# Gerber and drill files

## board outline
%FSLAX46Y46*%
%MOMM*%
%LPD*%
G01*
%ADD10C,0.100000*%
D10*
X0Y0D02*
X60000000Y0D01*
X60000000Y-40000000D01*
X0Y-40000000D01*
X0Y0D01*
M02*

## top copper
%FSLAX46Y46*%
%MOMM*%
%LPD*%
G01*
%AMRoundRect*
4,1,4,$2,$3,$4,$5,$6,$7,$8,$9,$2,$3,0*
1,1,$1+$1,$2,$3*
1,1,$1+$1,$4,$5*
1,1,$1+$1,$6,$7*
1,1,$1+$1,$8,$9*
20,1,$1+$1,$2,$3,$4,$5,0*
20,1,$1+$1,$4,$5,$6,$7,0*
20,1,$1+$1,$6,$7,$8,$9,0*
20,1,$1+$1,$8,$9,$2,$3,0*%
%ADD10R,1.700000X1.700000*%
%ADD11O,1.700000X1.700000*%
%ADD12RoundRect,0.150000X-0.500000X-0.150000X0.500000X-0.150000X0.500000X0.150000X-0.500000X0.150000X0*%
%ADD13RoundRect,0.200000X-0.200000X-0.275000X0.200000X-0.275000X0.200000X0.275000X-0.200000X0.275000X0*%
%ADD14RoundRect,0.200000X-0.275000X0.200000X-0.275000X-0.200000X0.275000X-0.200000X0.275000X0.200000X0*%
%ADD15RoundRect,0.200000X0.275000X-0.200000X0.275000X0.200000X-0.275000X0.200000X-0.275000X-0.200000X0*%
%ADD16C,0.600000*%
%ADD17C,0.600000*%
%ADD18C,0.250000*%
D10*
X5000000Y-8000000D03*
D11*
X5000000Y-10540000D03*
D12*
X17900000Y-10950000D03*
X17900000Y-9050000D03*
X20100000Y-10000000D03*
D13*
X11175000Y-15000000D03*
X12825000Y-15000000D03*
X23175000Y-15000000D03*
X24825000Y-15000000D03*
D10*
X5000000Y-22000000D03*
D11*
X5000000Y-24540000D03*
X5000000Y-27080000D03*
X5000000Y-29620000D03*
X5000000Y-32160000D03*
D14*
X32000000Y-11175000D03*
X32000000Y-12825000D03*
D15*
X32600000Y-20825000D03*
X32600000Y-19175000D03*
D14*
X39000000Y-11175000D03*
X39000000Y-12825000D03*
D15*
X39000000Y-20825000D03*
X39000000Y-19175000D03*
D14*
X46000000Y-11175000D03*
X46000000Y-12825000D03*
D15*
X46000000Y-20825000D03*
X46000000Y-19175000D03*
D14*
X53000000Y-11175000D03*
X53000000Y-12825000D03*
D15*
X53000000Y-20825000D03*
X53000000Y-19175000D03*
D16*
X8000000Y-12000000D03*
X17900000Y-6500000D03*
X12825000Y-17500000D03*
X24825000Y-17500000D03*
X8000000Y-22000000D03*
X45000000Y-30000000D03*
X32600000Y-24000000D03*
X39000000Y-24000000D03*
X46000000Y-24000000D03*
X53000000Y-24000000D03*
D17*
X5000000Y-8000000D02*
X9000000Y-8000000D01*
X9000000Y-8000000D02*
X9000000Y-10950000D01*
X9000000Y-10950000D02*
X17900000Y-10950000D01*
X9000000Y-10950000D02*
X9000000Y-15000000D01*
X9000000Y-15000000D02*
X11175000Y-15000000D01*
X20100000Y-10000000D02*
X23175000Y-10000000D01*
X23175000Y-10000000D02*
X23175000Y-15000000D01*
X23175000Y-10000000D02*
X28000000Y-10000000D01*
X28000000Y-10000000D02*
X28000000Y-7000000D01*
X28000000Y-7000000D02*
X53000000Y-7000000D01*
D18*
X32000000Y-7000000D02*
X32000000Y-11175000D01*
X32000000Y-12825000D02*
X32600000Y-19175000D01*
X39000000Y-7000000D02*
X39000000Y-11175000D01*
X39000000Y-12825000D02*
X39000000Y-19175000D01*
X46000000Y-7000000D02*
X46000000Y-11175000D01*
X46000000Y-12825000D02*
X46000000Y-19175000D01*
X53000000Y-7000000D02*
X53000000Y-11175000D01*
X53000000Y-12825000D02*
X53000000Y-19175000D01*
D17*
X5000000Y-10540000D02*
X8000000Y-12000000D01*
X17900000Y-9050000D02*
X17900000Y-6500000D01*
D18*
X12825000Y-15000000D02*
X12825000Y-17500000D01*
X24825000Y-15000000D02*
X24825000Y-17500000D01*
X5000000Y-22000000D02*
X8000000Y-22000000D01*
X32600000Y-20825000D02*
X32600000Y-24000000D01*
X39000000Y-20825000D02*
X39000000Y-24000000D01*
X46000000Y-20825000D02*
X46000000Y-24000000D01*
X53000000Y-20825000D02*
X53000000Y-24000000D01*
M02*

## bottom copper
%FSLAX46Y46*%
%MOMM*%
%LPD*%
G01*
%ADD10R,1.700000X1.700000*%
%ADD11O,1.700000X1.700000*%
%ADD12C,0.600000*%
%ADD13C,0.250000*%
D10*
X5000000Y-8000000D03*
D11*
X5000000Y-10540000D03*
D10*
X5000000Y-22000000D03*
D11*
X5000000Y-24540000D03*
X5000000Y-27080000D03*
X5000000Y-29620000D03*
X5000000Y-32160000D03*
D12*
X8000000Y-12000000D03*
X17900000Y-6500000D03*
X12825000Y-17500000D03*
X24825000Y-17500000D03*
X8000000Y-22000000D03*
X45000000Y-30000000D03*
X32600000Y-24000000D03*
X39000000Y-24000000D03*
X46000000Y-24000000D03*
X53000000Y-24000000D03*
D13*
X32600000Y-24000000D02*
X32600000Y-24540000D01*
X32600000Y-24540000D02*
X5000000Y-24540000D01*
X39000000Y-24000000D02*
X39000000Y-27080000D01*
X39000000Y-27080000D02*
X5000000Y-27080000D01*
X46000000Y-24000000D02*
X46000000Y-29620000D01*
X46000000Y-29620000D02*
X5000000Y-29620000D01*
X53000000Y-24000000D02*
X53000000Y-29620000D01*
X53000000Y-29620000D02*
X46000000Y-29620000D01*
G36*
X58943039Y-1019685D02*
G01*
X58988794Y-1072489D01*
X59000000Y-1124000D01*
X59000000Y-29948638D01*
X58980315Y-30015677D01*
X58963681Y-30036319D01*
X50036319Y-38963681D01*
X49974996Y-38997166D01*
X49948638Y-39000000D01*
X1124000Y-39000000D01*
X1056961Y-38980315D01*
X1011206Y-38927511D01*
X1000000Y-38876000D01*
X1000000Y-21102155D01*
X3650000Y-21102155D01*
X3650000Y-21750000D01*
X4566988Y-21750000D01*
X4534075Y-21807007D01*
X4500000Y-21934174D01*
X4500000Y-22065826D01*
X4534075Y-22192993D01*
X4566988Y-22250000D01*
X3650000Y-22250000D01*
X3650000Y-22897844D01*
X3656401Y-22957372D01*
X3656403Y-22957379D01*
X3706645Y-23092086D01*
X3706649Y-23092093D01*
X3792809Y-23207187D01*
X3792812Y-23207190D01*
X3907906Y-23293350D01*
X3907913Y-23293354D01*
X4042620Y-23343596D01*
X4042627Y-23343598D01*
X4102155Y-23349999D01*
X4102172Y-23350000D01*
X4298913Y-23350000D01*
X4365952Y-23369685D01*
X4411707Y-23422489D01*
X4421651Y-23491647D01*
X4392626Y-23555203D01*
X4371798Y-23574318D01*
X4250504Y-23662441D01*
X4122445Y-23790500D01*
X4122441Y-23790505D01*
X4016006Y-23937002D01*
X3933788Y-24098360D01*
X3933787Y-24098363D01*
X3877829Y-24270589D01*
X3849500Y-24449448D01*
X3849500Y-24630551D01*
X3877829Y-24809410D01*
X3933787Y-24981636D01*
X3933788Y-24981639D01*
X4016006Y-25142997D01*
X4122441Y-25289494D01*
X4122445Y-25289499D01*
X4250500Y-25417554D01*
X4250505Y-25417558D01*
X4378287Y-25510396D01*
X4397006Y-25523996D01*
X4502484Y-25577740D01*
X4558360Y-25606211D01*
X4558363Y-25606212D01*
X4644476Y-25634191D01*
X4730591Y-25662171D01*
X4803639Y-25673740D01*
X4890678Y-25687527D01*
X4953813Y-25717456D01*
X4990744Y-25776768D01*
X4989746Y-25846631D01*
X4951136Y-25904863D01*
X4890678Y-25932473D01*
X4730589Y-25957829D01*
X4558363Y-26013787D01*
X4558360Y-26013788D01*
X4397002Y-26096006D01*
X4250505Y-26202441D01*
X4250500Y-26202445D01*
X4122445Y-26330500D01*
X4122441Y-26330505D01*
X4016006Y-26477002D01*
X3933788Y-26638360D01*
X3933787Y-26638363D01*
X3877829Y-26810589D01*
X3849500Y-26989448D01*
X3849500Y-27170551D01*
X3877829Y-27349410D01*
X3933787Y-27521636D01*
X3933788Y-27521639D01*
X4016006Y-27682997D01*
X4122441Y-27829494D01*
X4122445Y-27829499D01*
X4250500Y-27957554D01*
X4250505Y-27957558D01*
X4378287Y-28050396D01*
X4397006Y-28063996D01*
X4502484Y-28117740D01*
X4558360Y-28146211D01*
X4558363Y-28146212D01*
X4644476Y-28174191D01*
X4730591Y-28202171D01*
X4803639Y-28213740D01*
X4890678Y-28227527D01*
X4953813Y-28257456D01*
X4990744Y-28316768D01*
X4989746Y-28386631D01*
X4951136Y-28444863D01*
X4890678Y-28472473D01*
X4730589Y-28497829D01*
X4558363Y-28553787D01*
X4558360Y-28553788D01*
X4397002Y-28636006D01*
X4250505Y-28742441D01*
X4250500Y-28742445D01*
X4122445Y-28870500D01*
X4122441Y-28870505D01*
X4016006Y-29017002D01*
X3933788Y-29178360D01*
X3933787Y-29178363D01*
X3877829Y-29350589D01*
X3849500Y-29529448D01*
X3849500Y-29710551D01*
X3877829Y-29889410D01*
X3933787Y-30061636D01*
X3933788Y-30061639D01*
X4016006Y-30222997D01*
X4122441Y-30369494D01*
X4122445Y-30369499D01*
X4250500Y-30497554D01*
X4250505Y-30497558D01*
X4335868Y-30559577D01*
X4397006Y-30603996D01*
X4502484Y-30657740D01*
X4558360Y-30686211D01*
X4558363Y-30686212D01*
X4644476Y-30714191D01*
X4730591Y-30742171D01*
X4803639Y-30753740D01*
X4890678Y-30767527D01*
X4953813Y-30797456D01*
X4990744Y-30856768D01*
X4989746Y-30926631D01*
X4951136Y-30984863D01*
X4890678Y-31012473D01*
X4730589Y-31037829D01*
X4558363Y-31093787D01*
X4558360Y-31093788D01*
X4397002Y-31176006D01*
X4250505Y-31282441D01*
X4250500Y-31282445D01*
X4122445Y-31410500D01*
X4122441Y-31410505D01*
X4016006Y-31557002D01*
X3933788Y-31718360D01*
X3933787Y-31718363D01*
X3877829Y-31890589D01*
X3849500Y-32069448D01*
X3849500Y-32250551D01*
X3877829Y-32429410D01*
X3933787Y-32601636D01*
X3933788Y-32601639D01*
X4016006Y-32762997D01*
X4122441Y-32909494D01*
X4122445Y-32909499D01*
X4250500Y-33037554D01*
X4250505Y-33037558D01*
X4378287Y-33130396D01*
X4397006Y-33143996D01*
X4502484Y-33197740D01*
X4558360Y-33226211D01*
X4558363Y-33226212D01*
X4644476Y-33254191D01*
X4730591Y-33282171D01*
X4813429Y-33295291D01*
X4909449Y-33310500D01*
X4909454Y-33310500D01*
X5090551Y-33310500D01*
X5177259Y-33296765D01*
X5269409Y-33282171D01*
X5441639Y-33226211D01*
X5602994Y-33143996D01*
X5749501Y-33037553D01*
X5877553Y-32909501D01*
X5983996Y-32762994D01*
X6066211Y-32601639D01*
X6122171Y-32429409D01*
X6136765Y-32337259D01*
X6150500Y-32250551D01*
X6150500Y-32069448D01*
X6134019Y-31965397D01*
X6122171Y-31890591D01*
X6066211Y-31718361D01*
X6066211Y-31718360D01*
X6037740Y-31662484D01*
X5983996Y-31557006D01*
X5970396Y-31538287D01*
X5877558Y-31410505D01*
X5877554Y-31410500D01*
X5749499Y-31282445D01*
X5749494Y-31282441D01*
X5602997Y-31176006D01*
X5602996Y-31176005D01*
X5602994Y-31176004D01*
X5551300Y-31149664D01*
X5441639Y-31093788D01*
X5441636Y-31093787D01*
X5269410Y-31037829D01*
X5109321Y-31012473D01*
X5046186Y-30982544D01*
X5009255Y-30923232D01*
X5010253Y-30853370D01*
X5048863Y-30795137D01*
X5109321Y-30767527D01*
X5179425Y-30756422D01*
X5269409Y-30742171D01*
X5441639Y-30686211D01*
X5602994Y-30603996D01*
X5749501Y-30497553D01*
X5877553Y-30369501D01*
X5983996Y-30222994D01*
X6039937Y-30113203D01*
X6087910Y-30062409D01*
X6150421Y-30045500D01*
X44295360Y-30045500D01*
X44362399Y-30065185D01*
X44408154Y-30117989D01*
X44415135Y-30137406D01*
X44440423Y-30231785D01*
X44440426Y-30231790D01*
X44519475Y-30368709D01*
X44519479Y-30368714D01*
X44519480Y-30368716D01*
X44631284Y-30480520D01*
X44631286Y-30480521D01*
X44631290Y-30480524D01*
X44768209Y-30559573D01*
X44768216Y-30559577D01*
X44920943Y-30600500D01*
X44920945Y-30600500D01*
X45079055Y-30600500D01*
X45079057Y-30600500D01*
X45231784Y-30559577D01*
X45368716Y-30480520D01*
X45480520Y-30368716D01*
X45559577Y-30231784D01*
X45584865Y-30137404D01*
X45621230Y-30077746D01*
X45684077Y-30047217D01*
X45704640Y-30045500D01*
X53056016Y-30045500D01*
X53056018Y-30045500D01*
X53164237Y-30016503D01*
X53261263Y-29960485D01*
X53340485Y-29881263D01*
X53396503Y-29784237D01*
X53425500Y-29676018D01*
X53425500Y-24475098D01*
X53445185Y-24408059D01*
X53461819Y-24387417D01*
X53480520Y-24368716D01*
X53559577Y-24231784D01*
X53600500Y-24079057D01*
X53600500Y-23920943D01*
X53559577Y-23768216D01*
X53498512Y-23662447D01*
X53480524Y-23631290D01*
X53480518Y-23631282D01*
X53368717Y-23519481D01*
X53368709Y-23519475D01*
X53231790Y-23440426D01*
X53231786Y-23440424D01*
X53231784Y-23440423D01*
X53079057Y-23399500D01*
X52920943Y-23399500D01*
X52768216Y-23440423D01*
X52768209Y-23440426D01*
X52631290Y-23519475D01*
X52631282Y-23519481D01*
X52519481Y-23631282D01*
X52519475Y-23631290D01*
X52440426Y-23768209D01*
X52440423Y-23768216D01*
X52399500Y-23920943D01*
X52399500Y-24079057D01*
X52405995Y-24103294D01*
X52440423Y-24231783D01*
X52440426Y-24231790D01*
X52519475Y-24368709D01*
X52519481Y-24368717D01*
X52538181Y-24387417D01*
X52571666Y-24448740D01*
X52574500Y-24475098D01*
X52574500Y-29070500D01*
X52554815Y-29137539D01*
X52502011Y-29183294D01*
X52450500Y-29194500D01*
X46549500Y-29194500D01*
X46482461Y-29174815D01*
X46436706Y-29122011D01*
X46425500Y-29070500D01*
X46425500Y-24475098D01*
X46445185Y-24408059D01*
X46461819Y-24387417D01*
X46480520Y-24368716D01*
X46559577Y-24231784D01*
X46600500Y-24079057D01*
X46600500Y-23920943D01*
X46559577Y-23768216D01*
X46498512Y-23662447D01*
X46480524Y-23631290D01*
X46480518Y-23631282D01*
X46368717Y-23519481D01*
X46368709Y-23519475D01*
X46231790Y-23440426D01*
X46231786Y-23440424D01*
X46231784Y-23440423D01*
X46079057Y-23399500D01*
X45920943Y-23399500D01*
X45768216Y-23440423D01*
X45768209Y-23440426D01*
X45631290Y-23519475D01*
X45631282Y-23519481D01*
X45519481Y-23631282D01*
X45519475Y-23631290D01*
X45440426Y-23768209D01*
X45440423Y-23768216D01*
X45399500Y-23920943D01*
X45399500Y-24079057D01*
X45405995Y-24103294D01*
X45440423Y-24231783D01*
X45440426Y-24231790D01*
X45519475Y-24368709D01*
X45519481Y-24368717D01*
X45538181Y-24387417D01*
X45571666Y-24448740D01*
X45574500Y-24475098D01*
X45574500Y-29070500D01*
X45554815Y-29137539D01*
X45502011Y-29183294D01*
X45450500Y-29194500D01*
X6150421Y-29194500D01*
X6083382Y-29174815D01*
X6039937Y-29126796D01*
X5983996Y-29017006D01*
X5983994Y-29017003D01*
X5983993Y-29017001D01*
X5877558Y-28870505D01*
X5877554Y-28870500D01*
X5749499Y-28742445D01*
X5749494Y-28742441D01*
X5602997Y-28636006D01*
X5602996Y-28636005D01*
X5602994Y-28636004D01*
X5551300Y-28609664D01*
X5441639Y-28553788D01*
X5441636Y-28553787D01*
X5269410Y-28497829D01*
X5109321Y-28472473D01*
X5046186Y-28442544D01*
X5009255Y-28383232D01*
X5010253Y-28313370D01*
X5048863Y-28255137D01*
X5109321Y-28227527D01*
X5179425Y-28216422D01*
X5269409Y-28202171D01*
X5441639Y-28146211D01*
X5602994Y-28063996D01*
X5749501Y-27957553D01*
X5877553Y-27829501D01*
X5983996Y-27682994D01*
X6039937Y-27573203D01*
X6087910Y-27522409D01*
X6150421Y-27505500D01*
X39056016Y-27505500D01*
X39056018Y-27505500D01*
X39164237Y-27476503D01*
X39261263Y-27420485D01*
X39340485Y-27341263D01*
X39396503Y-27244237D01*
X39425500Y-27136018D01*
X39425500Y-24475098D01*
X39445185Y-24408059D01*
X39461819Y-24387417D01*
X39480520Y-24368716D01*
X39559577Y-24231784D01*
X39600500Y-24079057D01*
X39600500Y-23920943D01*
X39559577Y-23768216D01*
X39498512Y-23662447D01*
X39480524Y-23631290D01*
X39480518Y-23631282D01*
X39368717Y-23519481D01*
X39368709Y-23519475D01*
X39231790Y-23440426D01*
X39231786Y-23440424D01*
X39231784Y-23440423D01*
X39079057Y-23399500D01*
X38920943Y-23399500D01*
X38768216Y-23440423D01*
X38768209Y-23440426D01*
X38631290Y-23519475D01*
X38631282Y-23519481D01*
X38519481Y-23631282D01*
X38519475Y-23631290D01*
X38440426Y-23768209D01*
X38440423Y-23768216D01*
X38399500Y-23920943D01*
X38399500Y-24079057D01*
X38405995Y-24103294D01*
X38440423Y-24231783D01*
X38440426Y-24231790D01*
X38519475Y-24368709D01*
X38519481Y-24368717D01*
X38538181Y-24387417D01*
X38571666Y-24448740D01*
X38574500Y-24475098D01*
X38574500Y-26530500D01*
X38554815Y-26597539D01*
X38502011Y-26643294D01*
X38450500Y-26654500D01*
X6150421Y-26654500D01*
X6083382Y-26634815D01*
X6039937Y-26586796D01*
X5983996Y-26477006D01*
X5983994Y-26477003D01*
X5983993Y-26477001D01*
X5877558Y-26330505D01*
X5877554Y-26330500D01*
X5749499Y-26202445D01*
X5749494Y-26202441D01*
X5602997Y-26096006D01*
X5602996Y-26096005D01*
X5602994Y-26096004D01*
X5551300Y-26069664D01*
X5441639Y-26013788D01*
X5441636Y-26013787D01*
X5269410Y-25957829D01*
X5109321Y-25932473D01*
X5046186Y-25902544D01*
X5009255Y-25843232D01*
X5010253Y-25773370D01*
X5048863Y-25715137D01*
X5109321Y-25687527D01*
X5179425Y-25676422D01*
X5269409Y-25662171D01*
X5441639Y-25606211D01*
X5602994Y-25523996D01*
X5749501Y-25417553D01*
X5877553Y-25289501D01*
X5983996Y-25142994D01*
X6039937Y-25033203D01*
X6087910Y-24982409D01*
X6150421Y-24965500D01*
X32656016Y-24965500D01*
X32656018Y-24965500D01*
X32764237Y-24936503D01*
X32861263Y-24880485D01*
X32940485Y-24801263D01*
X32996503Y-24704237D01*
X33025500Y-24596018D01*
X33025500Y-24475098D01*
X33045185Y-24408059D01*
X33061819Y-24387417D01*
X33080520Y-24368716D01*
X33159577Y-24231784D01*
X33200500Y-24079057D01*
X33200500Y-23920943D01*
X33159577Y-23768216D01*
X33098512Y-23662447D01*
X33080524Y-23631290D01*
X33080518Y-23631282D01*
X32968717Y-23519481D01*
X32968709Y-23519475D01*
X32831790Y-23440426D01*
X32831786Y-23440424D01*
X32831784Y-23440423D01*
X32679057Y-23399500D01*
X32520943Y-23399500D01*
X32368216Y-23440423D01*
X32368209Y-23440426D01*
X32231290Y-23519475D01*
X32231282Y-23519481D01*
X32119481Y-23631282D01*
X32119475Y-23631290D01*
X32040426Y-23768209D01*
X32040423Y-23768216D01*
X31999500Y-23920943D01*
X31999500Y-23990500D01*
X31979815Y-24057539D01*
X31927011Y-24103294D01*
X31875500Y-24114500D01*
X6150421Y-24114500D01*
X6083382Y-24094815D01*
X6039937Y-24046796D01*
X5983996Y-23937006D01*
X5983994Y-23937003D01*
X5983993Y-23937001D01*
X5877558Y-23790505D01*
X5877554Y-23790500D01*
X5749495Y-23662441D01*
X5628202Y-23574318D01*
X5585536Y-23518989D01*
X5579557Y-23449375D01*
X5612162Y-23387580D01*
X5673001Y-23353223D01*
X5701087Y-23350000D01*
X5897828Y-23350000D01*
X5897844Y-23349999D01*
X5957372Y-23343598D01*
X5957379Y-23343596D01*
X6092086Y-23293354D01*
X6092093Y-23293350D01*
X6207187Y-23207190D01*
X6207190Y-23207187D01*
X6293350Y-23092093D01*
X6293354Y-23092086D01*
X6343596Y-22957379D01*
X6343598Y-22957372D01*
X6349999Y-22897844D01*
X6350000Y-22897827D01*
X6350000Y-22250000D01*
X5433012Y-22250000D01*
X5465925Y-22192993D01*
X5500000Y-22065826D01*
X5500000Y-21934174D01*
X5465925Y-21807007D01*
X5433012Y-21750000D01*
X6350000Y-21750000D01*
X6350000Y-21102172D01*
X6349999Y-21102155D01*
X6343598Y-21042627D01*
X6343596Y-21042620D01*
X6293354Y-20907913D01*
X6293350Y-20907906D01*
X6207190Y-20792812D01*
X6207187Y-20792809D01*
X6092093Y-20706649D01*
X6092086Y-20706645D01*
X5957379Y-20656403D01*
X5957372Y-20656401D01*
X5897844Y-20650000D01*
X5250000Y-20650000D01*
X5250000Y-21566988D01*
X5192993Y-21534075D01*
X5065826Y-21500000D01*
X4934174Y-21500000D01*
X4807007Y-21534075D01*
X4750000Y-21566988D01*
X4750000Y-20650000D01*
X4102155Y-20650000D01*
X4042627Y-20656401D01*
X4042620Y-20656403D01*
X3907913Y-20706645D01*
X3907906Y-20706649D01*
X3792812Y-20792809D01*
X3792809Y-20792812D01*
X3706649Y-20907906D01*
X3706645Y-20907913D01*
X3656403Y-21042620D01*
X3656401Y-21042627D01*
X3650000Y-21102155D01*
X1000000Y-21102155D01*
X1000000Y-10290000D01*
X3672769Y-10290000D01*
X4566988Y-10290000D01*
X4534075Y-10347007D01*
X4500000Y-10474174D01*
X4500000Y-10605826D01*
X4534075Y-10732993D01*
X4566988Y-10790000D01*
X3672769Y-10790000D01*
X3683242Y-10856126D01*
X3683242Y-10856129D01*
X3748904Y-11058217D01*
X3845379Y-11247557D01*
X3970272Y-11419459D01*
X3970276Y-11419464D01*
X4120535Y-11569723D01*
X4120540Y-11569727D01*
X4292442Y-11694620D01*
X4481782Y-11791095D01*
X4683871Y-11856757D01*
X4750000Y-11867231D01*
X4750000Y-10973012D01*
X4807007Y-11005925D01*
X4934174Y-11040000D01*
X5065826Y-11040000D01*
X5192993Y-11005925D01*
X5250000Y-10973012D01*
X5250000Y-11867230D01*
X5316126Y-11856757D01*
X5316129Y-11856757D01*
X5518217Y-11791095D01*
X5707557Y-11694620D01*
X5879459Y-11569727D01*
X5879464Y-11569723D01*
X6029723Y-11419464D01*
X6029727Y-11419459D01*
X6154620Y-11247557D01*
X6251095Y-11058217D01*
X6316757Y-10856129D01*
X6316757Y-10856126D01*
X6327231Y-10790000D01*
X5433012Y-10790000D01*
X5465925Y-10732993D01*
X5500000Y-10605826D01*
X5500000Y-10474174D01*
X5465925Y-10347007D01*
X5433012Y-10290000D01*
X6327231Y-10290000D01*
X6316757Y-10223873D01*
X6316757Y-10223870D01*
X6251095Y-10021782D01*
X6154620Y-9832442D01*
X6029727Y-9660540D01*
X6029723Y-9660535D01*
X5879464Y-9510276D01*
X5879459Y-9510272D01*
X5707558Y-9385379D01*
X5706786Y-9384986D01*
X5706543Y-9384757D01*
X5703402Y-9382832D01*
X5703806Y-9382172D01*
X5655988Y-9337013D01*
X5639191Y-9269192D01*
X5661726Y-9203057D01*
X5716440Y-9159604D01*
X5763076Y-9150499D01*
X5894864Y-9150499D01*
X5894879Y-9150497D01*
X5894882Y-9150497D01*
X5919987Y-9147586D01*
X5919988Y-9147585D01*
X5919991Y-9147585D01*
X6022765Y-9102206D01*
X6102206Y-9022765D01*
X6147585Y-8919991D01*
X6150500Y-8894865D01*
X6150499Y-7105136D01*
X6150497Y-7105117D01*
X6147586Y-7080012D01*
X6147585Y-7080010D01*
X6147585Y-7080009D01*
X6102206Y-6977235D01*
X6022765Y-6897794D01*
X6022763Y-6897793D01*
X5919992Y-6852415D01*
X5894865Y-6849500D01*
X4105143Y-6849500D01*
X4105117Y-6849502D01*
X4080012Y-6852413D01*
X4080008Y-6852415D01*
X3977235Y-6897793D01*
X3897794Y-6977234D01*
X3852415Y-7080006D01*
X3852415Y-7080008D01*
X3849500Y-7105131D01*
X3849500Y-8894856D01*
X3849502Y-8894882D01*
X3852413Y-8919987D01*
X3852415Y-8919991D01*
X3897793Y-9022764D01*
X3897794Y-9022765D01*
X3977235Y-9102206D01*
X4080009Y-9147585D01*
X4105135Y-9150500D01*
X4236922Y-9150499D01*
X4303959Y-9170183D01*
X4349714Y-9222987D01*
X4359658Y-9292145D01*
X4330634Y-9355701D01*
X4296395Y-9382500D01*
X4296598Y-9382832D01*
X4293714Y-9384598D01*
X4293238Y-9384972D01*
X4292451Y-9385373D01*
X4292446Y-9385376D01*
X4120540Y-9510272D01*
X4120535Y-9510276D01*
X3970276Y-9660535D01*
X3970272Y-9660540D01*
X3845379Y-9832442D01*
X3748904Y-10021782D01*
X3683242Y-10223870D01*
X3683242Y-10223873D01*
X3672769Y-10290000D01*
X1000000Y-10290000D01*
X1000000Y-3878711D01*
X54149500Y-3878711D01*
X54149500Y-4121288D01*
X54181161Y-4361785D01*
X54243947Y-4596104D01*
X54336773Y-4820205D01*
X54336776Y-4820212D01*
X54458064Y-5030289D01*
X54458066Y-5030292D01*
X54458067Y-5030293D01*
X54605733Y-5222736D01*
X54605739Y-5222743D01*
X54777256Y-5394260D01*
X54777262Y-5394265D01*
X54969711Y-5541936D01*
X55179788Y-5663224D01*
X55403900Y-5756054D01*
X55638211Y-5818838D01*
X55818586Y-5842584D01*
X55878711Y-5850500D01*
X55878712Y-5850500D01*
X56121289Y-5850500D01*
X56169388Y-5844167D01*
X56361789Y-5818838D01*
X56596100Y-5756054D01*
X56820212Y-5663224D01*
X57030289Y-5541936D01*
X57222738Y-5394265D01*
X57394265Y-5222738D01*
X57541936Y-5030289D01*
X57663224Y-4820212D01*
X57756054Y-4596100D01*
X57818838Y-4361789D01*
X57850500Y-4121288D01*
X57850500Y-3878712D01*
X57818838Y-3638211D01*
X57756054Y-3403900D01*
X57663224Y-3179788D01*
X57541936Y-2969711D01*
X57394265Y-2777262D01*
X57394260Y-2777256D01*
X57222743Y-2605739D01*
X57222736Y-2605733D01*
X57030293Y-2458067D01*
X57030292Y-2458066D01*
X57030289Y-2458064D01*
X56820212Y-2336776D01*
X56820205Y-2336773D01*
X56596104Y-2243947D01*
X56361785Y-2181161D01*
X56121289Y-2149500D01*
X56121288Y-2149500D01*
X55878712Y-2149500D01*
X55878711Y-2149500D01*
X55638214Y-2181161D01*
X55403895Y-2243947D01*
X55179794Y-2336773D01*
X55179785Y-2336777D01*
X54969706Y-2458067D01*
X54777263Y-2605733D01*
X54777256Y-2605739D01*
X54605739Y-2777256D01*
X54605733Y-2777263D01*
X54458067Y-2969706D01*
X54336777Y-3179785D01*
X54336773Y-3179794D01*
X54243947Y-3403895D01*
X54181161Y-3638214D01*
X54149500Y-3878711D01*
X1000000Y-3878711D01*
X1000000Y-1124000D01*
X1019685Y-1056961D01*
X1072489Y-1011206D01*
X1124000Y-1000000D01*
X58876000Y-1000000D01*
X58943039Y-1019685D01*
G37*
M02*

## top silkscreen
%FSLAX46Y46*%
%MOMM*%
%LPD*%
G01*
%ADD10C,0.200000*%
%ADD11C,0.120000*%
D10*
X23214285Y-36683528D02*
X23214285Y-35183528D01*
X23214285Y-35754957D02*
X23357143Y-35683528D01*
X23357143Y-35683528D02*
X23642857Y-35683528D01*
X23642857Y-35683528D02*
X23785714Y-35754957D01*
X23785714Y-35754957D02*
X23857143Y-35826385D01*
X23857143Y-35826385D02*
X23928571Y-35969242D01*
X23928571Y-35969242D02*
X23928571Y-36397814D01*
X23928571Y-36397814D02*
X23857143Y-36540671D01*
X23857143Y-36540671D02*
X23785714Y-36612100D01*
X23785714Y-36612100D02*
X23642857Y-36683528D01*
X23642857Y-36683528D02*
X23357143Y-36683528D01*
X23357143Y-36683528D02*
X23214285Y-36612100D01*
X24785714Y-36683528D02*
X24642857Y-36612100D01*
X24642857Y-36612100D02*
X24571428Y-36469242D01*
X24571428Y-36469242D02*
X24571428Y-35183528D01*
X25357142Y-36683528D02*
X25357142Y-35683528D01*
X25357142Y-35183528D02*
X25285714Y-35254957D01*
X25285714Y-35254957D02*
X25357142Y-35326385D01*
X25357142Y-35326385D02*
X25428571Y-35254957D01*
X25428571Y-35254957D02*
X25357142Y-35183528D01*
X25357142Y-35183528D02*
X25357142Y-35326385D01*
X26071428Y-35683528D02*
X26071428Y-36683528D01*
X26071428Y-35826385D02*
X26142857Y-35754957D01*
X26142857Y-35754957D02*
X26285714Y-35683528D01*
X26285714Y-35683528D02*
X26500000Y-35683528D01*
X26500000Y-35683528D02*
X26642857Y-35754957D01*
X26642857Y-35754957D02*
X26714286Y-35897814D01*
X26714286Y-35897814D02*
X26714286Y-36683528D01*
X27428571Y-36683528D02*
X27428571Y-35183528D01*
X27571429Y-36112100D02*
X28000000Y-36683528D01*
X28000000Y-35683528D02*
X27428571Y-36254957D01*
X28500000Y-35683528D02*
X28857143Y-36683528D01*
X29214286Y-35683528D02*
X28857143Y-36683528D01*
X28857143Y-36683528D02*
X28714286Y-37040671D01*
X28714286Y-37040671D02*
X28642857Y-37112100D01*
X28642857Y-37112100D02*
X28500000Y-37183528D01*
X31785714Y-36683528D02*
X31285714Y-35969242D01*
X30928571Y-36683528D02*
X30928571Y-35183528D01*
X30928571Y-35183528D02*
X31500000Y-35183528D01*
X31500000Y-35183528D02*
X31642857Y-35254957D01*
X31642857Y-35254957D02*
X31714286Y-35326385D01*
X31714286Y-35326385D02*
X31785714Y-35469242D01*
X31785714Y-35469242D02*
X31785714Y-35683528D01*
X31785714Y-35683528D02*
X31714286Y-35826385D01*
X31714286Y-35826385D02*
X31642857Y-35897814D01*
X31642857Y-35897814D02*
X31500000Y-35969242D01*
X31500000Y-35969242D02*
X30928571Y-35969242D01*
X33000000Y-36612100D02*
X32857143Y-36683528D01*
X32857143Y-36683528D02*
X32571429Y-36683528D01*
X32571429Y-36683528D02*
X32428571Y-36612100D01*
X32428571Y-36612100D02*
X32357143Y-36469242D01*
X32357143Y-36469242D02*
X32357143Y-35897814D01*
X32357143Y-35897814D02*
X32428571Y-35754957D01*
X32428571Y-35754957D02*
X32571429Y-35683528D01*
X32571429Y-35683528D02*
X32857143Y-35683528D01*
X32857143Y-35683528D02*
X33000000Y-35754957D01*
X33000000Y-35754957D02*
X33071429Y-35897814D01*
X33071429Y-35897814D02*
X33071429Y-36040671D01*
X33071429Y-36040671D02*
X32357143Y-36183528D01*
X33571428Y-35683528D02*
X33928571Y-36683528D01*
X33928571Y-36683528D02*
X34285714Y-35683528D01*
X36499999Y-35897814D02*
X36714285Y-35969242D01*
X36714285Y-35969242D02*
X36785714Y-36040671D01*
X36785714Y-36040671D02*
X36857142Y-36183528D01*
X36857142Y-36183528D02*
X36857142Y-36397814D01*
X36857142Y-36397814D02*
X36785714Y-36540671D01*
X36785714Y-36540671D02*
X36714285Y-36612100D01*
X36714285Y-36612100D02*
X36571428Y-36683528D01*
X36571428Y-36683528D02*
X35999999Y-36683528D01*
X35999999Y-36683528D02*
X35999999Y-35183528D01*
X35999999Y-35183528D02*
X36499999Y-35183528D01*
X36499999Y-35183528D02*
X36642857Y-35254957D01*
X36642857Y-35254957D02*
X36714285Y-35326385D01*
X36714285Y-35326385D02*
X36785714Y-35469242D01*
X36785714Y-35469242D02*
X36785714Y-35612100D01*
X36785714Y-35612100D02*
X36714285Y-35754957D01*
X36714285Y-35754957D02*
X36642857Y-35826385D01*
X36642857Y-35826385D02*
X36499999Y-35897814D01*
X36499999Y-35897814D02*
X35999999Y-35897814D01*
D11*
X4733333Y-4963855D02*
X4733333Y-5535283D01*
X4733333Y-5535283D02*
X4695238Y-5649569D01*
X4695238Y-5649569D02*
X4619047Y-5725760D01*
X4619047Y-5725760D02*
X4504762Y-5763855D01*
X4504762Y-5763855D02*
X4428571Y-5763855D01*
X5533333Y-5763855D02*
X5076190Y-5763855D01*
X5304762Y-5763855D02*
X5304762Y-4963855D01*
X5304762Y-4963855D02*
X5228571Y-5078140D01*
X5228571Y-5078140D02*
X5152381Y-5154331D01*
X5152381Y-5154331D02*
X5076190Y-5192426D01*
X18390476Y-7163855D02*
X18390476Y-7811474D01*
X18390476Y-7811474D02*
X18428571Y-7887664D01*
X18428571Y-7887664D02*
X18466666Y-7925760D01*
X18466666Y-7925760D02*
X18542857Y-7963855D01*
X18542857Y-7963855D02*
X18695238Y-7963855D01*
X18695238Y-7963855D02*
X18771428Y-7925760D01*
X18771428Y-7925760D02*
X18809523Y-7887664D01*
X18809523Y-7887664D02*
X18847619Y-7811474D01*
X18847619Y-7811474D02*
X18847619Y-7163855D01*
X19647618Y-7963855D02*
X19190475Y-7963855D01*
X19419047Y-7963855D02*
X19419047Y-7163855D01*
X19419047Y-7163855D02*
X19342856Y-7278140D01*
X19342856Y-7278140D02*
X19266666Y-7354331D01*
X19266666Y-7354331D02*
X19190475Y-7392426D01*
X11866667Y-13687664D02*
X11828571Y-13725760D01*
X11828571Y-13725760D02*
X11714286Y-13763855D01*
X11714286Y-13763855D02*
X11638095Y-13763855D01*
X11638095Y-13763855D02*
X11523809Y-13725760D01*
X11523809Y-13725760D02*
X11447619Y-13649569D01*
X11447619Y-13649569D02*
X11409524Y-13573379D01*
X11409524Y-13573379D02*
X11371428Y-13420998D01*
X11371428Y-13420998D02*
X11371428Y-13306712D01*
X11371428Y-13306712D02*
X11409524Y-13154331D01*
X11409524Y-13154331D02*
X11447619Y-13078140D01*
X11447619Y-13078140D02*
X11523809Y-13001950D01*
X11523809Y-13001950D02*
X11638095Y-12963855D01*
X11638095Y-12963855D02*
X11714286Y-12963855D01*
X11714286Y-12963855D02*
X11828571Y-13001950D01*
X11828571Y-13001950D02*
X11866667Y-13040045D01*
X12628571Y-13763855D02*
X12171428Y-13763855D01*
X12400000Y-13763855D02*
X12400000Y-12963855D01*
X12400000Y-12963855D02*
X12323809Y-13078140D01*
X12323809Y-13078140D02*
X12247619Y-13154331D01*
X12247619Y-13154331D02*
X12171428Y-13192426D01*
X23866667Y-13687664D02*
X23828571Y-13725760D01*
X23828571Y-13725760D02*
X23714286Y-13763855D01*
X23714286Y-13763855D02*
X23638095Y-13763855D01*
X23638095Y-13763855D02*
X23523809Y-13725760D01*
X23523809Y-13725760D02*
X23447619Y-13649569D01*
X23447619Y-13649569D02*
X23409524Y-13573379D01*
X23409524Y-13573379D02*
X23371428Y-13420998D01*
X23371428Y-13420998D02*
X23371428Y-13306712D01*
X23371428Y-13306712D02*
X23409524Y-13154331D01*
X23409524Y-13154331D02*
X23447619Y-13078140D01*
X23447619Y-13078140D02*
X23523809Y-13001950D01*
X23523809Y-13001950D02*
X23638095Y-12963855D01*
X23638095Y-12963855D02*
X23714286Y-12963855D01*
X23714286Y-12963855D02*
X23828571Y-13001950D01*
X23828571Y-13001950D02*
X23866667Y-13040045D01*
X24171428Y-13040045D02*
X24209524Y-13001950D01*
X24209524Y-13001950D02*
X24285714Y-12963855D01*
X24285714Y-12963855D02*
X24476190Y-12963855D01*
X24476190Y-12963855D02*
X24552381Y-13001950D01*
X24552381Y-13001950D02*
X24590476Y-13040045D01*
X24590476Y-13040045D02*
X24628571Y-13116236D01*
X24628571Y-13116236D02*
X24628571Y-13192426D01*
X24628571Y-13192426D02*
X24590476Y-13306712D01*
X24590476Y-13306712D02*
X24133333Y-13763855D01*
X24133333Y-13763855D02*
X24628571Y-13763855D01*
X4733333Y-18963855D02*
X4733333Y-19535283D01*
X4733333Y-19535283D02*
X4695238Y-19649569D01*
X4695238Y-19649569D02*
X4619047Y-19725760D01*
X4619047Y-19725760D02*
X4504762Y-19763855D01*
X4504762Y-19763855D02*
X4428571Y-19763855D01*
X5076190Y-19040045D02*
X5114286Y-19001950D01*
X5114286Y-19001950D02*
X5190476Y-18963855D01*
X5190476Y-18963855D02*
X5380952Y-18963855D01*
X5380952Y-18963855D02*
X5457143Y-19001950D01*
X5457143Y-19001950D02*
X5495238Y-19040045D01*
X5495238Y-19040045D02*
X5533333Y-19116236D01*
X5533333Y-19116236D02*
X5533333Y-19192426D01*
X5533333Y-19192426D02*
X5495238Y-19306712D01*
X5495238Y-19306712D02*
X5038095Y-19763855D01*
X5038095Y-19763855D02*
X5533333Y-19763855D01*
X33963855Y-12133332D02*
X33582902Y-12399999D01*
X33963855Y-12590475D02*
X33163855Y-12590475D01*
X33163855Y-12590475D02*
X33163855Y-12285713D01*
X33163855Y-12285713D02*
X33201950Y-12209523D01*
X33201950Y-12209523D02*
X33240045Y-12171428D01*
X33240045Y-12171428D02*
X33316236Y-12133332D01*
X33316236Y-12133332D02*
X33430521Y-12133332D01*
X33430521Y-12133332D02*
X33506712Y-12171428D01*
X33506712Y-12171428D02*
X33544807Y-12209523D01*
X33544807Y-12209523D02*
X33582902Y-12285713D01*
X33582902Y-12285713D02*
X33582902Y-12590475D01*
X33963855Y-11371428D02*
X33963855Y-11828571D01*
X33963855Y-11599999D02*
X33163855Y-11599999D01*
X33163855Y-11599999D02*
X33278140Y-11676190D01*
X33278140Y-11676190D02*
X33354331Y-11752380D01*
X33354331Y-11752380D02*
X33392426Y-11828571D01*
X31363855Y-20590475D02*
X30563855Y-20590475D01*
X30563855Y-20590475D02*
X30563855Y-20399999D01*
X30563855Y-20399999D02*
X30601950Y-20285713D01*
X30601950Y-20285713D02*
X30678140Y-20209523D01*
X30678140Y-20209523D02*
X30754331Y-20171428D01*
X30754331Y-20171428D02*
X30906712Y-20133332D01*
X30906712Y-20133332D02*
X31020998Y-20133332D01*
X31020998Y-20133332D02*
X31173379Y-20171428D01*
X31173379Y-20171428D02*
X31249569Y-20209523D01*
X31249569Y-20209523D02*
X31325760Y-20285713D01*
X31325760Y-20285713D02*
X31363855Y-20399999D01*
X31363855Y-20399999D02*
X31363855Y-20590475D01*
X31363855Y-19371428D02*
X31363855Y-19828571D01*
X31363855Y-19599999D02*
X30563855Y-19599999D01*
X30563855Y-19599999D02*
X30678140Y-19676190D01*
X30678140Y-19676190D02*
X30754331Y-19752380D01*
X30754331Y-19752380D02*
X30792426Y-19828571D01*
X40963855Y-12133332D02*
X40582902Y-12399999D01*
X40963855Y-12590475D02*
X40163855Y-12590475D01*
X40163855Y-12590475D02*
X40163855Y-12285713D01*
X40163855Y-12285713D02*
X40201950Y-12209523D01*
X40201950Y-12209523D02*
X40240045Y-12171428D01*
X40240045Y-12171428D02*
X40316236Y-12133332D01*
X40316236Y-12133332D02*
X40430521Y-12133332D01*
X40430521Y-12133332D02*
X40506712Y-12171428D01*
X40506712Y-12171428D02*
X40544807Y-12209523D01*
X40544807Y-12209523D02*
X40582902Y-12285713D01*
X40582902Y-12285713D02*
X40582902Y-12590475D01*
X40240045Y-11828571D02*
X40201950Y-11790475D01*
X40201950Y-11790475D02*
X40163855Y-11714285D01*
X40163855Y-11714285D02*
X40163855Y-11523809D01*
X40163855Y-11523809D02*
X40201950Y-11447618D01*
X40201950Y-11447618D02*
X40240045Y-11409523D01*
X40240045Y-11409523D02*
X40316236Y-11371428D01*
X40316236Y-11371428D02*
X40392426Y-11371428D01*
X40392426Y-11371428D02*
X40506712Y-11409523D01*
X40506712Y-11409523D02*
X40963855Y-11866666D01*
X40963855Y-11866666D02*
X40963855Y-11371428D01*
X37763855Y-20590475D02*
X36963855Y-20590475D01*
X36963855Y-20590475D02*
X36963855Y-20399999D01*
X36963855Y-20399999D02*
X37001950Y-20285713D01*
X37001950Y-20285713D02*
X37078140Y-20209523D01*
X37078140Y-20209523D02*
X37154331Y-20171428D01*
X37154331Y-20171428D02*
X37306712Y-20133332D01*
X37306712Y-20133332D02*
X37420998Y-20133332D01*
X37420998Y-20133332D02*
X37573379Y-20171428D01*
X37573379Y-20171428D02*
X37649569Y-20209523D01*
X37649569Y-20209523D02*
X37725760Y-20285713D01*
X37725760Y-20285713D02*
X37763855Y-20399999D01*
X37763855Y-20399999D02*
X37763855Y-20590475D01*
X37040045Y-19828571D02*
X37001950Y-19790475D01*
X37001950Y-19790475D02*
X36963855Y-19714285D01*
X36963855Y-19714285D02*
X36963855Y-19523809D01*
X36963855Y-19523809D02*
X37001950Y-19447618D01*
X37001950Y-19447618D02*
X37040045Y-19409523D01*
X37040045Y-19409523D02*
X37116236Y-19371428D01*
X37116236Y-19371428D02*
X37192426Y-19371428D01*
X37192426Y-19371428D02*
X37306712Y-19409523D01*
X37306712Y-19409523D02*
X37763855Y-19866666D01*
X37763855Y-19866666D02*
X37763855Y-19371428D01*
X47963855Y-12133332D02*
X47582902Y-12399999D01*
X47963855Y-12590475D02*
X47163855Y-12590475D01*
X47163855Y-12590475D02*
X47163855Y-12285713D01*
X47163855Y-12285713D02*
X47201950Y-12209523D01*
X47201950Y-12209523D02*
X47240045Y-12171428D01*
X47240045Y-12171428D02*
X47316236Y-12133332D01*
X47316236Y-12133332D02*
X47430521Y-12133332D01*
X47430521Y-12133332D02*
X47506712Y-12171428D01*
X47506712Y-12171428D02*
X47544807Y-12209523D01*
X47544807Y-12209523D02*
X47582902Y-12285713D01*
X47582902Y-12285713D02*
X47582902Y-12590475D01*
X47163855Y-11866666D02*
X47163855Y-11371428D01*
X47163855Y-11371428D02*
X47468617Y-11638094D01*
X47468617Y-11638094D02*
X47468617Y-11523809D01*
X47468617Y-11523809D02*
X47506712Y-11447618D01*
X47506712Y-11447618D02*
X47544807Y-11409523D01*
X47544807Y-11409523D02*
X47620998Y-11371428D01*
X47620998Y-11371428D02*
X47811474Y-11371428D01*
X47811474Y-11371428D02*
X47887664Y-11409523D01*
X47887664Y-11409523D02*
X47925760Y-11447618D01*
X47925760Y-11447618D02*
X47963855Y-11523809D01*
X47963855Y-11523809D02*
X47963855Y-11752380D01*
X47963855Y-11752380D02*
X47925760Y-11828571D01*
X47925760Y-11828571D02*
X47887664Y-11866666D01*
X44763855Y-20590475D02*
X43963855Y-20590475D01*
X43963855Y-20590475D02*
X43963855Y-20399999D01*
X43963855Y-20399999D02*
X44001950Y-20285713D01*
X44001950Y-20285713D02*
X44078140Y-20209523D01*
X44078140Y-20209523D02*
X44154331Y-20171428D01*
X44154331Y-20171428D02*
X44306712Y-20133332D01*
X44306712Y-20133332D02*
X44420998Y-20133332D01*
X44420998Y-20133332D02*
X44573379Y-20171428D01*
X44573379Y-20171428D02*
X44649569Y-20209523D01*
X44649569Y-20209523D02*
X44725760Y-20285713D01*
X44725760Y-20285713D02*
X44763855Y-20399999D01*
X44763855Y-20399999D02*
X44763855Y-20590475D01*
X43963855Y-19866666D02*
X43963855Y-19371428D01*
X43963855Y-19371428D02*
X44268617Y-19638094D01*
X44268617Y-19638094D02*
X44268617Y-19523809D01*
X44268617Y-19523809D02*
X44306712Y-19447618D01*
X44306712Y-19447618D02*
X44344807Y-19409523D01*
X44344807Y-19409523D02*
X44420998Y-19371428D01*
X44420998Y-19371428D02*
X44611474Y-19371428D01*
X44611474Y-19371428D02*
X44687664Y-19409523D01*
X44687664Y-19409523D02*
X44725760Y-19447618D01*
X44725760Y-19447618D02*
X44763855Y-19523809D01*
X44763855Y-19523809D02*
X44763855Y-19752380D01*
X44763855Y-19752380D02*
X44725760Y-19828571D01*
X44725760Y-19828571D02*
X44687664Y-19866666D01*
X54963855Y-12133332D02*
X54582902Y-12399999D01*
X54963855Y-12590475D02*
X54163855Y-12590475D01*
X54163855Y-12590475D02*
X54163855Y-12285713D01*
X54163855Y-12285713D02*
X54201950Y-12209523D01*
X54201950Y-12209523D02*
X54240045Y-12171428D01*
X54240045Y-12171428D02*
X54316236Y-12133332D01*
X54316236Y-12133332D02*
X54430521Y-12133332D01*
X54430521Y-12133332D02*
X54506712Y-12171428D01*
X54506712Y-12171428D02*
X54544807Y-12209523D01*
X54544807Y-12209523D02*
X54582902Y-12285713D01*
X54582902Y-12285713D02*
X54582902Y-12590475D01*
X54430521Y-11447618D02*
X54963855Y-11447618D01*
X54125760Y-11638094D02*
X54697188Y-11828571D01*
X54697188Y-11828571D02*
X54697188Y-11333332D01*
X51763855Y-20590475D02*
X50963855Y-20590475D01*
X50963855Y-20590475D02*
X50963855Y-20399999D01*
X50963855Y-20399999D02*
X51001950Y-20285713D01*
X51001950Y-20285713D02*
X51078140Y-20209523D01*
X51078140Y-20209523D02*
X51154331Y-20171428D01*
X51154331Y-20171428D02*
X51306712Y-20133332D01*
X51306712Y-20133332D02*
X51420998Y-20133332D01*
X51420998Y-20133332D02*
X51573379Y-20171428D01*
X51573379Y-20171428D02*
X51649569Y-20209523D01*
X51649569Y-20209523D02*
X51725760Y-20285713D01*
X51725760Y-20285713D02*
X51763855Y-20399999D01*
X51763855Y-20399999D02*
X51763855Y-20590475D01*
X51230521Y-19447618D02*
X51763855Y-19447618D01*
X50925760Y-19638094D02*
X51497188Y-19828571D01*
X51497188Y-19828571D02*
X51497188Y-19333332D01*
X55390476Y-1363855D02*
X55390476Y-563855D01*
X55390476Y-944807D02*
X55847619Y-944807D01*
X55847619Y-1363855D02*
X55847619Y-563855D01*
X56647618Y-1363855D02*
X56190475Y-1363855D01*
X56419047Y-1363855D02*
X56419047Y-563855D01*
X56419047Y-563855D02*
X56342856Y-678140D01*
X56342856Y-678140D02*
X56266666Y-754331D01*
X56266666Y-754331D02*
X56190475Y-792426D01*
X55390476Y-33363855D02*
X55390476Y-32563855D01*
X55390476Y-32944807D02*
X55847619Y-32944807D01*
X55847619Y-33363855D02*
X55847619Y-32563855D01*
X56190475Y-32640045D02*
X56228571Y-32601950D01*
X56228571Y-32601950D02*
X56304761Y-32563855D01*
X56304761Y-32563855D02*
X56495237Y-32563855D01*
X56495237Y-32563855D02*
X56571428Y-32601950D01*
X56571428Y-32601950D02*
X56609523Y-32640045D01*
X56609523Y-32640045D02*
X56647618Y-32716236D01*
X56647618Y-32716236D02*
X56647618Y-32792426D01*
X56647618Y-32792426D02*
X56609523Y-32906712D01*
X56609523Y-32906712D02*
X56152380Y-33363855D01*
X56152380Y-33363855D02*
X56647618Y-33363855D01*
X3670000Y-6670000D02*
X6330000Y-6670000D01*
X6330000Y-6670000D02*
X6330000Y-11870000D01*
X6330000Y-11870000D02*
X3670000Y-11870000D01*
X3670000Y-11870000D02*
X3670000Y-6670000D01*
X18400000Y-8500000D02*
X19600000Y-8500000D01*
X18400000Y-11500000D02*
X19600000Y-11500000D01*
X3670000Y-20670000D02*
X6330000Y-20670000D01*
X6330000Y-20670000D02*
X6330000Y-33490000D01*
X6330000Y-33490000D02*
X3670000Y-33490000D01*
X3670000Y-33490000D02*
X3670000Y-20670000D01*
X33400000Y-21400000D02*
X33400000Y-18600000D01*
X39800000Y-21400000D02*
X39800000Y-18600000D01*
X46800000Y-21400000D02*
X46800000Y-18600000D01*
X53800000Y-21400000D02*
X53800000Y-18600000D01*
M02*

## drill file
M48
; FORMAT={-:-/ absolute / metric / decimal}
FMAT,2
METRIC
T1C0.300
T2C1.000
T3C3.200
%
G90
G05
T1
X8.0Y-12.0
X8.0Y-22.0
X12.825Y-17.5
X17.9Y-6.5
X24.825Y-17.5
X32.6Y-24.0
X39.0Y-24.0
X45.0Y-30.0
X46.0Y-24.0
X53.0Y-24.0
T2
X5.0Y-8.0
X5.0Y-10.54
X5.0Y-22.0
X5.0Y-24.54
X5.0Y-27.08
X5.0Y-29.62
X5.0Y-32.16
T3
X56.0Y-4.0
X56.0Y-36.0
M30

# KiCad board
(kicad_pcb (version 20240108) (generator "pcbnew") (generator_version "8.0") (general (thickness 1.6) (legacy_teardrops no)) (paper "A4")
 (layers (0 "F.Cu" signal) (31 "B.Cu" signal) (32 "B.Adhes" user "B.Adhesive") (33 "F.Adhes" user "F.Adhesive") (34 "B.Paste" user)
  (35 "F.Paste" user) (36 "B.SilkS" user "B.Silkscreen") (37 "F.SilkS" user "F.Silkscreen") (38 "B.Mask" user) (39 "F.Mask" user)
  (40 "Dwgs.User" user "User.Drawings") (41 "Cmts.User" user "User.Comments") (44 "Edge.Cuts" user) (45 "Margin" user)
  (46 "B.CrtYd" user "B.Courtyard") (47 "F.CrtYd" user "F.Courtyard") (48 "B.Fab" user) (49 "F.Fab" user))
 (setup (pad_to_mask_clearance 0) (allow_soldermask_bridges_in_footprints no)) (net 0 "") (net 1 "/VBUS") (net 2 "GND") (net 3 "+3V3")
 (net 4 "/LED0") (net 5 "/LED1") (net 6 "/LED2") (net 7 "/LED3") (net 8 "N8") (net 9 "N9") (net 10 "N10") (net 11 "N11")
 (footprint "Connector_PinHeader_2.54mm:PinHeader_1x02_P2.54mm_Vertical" (layer "F.Cu") (at 5 8)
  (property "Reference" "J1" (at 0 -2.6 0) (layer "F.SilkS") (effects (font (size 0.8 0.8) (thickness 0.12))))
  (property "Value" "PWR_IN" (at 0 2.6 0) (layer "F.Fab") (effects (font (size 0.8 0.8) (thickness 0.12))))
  (fp_line (start -1.33 -1.33) (end 1.33 -1.33) (stroke (width 0.12) (type solid)) (layer "F.SilkS"))
  (fp_line (start 1.33 -1.33) (end 1.33 3.87) (stroke (width 0.12) (type solid)) (layer "F.SilkS"))
  (fp_line (start 1.33 3.87) (end -1.33 3.87) (stroke (width 0.12) (type solid)) (layer "F.SilkS"))
  (fp_line (start -1.33 3.87) (end -1.33 -1.33) (stroke (width 0.12) (type solid)) (layer "F.SilkS"))
  (pad "1" thru_hole rect (at 0 0) (size 1.7 1.7) (drill 1) (layers "*.Cu" "*.Mask") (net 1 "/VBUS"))
  (pad "2" thru_hole oval (at 0 2.54) (size 1.7 1.7) (drill 1) (layers "*.Cu" "*.Mask") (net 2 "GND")))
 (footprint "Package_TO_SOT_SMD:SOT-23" (layer "F.Cu") (at 19 10)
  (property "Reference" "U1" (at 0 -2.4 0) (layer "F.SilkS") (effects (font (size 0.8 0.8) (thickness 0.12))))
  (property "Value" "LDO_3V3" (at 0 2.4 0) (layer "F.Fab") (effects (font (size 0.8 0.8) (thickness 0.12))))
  (fp_line (start -0.6 -1.5) (end 0.6 -1.5) (stroke (width 0.12) (type solid)) (layer "F.SilkS"))
  (fp_line (start -0.6 1.5) (end 0.6 1.5) (stroke (width 0.12) (type solid)) (layer "F.SilkS"))
  (pad "1" smd roundrect (at -1.1 0.95) (size 1.3 0.6) (layers "F.Cu" "F.Paste" "F.Mask") (roundrect_rratio 0.25) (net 1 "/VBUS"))
  (pad "2" smd roundrect (at -1.1 -0.95) (size 1.3 0.6) (layers "F.Cu" "F.Paste" "F.Mask") (roundrect_rratio 0.25) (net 2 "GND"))
  (pad "3" smd roundrect (at 1.1 0) (size 1.3 0.6) (layers "F.Cu" "F.Paste" "F.Mask") (roundrect_rratio 0.25) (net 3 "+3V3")))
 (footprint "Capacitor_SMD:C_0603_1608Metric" (layer "F.Cu") (at 12 15)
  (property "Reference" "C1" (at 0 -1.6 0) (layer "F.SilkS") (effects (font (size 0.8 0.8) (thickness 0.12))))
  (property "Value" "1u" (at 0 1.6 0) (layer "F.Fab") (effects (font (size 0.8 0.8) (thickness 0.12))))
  (pad "1" smd roundrect (at -0.825 0) (size 0.8 0.95) (layers "F.Cu" "F.Paste" "F.Mask") (roundrect_rratio 0.25) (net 1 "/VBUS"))
  (pad "2" smd roundrect (at 0.825 0) (size 0.8 0.95) (layers "F.Cu" "F.Paste" "F.Mask") (roundrect_rratio 0.25) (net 2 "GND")))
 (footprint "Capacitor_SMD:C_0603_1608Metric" (layer "F.Cu") (at 24 15)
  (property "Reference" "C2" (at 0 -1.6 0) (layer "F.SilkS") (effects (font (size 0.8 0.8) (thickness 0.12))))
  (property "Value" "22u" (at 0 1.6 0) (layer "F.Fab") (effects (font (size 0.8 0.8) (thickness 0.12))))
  (pad "1" smd roundrect (at -0.825 0) (size 0.8 0.95) (layers "F.Cu" "F.Paste" "F.Mask") (roundrect_rratio 0.25) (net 3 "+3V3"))
  (pad "2" smd roundrect (at 0.825 0) (size 0.8 0.95) (layers "F.Cu" "F.Paste" "F.Mask") (roundrect_rratio 0.25) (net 2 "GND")))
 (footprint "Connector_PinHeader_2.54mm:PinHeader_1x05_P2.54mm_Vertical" (layer "F.Cu") (at 5 22)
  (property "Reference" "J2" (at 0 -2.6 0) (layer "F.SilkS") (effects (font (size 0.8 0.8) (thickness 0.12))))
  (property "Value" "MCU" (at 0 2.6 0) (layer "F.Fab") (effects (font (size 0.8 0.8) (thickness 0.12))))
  (fp_line (start -1.33 -1.33) (end 1.33 -1.33) (stroke (width 0.12) (type solid)) (layer "F.SilkS"))
  (fp_line (start 1.33 -1.33) (end 1.33 11.49) (stroke (width 0.12) (type solid)) (layer "F.SilkS"))
  (fp_line (start 1.33 11.49) (end -1.33 11.49) (stroke (width 0.12) (type solid)) (layer "F.SilkS"))
  (fp_line (start -1.33 11.49) (end -1.33 -1.33) (stroke (width 0.12) (type solid)) (layer "F.SilkS"))
  (pad "1" thru_hole rect (at 0 0) (size 1.7 1.7) (drill 1) (layers "*.Cu" "*.Mask") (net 2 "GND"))
  (pad "2" thru_hole oval (at 0 2.54) (size 1.7 1.7) (drill 1) (layers "*.Cu" "*.Mask") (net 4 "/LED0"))
  (pad "3" thru_hole oval (at 0 5.08) (size 1.7 1.7) (drill 1) (layers "*.Cu" "*.Mask") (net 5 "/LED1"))
  (pad "4" thru_hole oval (at 0 7.62) (size 1.7 1.7) (drill 1) (layers "*.Cu" "*.Mask") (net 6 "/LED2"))
  (pad "5" thru_hole oval (at 0 10.16) (size 1.7 1.7) (drill 1) (layers "*.Cu" "*.Mask") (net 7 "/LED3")))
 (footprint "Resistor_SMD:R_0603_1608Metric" (layer "F.Cu") (at 32 12 270)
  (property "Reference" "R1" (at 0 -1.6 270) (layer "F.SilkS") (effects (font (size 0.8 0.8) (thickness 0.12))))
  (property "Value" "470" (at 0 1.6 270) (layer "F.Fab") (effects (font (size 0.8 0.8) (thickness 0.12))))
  (pad "1" smd roundrect (at -0.825 0 270) (size 0.8 0.95) (layers "F.Cu" "F.Paste" "F.Mask") (roundrect_rratio 0.25) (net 3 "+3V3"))
  (pad "2" smd roundrect (at 0.825 0 270) (size 0.8 0.95) (layers "F.Cu" "F.Paste" "F.Mask") (roundrect_rratio 0.25) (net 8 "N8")))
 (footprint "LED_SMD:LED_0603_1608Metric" (layer "F.Cu") (at 32.6 20 90)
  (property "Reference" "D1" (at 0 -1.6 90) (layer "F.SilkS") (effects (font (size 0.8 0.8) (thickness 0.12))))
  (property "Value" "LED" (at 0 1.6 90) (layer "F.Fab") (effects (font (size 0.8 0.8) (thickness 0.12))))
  (fp_line (start -1.4 0.8) (end 1.4 0.8) (stroke (width 0.12) (type solid)) (layer "F.SilkS"))
  (pad "1" smd roundrect (at -0.825 0 90) (size 0.8 0.95) (layers "F.Cu" "F.Paste" "F.Mask") (roundrect_rratio 0.25) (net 4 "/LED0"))
  (pad "2" smd roundrect (at 0.825 0 90) (size 0.8 0.95) (layers "F.Cu" "F.Paste" "F.Mask") (roundrect_rratio 0.25) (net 8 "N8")))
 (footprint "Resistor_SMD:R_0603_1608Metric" (layer "F.Cu") (at 39 12 270)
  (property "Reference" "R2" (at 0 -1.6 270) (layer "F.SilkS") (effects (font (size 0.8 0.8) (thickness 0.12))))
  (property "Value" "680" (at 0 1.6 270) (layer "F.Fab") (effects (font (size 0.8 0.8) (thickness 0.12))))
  (pad "1" smd roundrect (at -0.825 0 270) (size 0.8 0.95) (layers "F.Cu" "F.Paste" "F.Mask") (roundrect_rratio 0.25) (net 3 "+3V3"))
  (pad "2" smd roundrect (at 0.825 0 270) (size 0.8 0.95) (layers "F.Cu" "F.Paste" "F.Mask") (roundrect_rratio 0.25) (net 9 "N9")))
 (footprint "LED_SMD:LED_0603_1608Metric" (layer "F.Cu") (at 39 20 90)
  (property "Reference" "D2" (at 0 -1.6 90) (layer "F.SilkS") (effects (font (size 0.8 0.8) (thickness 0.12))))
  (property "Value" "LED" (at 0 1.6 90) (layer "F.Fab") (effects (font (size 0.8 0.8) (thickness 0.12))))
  (fp_line (start -1.4 0.8) (end 1.4 0.8) (stroke (width 0.12) (type solid)) (layer "F.SilkS"))
  (pad "1" smd roundrect (at -0.825 0 90) (size 0.8 0.95) (layers "F.Cu" "F.Paste" "F.Mask") (roundrect_rratio 0.25) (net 5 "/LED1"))
  (pad "2" smd roundrect (at 0.825 0 90) (size 0.8 0.95) (layers "F.Cu" "F.Paste" "F.Mask") (roundrect_rratio 0.25) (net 9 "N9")))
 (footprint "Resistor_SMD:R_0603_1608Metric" (layer "F.Cu") (at 46 12 270)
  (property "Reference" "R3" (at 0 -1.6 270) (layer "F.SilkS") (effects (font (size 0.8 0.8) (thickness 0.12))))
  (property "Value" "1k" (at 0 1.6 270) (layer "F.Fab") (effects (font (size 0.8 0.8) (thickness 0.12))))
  (pad "1" smd roundrect (at -0.825 0 270) (size 0.8 0.95) (layers "F.Cu" "F.Paste" "F.Mask") (roundrect_rratio 0.25) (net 3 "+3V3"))
  (pad "2" smd roundrect (at 0.825 0 270) (size 0.8 0.95) (layers "F.Cu" "F.Paste" "F.Mask") (roundrect_rratio 0.25) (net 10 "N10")))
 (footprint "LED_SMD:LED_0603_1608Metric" (layer "F.Cu") (at 46 20 90)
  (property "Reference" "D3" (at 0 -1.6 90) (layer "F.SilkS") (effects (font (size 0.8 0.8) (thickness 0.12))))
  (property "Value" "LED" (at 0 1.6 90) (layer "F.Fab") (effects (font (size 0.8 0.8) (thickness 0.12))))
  (fp_line (start -1.4 0.8) (end 1.4 0.8) (stroke (width 0.12) (type solid)) (layer "F.SilkS"))
  (pad "1" smd roundrect (at -0.825 0 90) (size 0.8 0.95) (layers "F.Cu" "F.Paste" "F.Mask") (roundrect_rratio 0.25) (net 6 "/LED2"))
  (pad "2" smd roundrect (at 0.825 0 90) (size 0.8 0.95) (layers "F.Cu" "F.Paste" "F.Mask") (roundrect_rratio 0.25) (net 10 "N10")))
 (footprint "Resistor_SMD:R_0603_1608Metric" (layer "F.Cu") (at 53 12 270)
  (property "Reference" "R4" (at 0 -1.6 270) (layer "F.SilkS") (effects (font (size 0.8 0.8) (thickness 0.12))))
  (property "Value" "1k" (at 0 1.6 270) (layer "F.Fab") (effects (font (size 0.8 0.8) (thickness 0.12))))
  (pad "1" smd roundrect (at -0.825 0 270) (size 0.8 0.95) (layers "F.Cu" "F.Paste" "F.Mask") (roundrect_rratio 0.25) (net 3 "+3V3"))
  (pad "2" smd roundrect (at 0.825 0 270) (size 0.8 0.95) (layers "F.Cu" "F.Paste" "F.Mask") (roundrect_rratio 0.25) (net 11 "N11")))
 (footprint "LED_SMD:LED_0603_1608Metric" (layer "F.Cu") (at 53 20 90)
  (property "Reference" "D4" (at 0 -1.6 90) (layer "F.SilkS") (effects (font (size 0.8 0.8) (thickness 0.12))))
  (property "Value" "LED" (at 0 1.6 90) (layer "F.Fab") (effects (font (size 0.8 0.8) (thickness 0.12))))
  (fp_line (start -1.4 0.8) (end 1.4 0.8) (stroke (width 0.12) (type solid)) (layer "F.SilkS"))
  (pad "1" smd roundrect (at -0.825 0 90) (size 0.8 0.95) (layers "F.Cu" "F.Paste" "F.Mask") (roundrect_rratio 0.25) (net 6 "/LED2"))
  (pad "2" smd roundrect (at 0.825 0 90) (size 0.8 0.95) (layers "F.Cu" "F.Paste" "F.Mask") (roundrect_rratio 0.25) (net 11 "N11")))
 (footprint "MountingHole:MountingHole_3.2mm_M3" (layer "F.Cu") (at 56 4)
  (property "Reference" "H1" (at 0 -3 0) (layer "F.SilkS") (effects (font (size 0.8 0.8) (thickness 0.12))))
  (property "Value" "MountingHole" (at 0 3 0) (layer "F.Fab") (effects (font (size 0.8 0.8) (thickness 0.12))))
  (pad "" np_thru_hole circle (at 0 0) (size 3.2 3.2) (drill 3.2) (layers "*.Cu" "*.Mask")))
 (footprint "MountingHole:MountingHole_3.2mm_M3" (layer "F.Cu") (at 56 36)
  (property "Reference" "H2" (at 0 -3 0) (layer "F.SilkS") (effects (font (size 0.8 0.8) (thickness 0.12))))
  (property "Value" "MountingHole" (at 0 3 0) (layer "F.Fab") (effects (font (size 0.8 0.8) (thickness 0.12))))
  (pad "" np_thru_hole circle (at 0 0) (size 3.2 3.2) (drill 3.2) (layers "*.Cu" "*.Mask")))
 (segment (start 5 8) (end 9 8) (width 0.6) (layer "F.Cu") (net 1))
 (segment (start 9 8) (end 9 10.95) (width 0.6) (layer "F.Cu") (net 1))
 (segment (start 9 10.95) (end 17.9 10.95) (width 0.6) (layer "F.Cu") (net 1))
 (segment (start 9 10.95) (end 9 15) (width 0.6) (layer "F.Cu") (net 1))
 (segment (start 9 15) (end 11.175 15) (width 0.6) (layer "F.Cu") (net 1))
 (segment (start 20.1 10) (end 23.175 10) (width 0.6) (layer "F.Cu") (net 3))
 (segment (start 23.175 10) (end 23.175 15) (width 0.6) (layer "F.Cu") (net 3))
 (segment (start 23.175 10) (end 28 10) (width 0.6) (layer "F.Cu") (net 3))
 (segment (start 28 10) (end 28 7) (width 0.6) (layer "F.Cu") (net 3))
 (segment (start 28 7) (end 53 7) (width 0.6) (layer "F.Cu") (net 3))
 (segment (start 32 7) (end 32 11.175) (width 0.25) (layer "F.Cu") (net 3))
 (segment (start 32 12.825) (end 32.6 19.175) (width 0.25) (layer "F.Cu") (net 8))
 (segment (start 39 7) (end 39 11.175) (width 0.25) (layer "F.Cu") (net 3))
 (segment (start 39 12.825) (end 39 19.175) (width 0.25) (layer "F.Cu") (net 9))
 (segment (start 46 7) (end 46 11.175) (width 0.25) (layer "F.Cu") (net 3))
 (segment (start 46 12.825) (end 46 19.175) (width 0.25) (layer "F.Cu") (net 10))
 (segment (start 53 7) (end 53 11.175) (width 0.25) (layer "F.Cu") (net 3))
 (segment (start 53 12.825) (end 53 19.175) (width 0.25) (layer "F.Cu") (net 11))
 (segment (start 5 10.54) (end 8 12) (width 0.6) (layer "F.Cu") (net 2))
 (via (at 8 12) (size 0.6) (drill 0.3) (layers "F.Cu" "B.Cu") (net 2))
 (segment (start 17.9 9.05) (end 17.9 6.5) (width 0.6) (layer "F.Cu") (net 2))
 (via (at 17.9 6.5) (size 0.6) (drill 0.3) (layers "F.Cu" "B.Cu") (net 2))
 (segment (start 12.825 15) (end 12.825 17.5) (width 0.25) (layer "F.Cu") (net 2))
 (via (at 12.825 17.5) (size 0.6) (drill 0.3) (layers "F.Cu" "B.Cu") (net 2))
 (segment (start 24.825 15) (end 24.825 17.5) (width 0.25) (layer "F.Cu") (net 2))
 (via (at 24.825 17.5) (size 0.6) (drill 0.3) (layers "F.Cu" "B.Cu") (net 2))
 (segment (start 5 22) (end 8 22) (width 0.25) (layer "F.Cu") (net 2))
 (via (at 8 22) (size 0.6) (drill 0.3) (layers "F.Cu" "B.Cu") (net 2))
 (via (at 45 30) (size 0.6) (drill 0.3) (layers "F.Cu" "B.Cu") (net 2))
 (segment (start 32.6 20.825) (end 32.6 24) (width 0.25) (layer "F.Cu") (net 4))
 (via (at 32.6 24) (size 0.6) (drill 0.3) (layers "F.Cu" "B.Cu") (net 4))
 (segment (start 32.6 24) (end 32.6 24.54) (width 0.25) (layer "B.Cu") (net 4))
 (segment (start 32.6 24.54) (end 5 24.54) (width 0.25) (layer "B.Cu") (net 4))
 (segment (start 39 20.825) (end 39 24) (width 0.25) (layer "F.Cu") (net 5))
 (via (at 39 24) (size 0.6) (drill 0.3) (layers "F.Cu" "B.Cu") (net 5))
 (segment (start 39 24) (end 39 27.08) (width 0.25) (layer "B.Cu") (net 5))
 (segment (start 39 27.08) (end 5 27.08) (width 0.25) (layer "B.Cu") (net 5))
 (segment (start 46 20.825) (end 46 24) (width 0.25) (layer "F.Cu") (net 6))
 (via (at 46 24) (size 0.6) (drill 0.3) (layers "F.Cu" "B.Cu") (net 6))
 (segment (start 46 24) (end 46 29.62) (width 0.25) (layer "B.Cu") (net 6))
 (segment (start 46 29.62) (end 5 29.62) (width 0.25) (layer "B.Cu") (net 6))
 (segment (start 53 20.825) (end 53 24) (width 0.25) (layer "F.Cu") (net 6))
 (via (at 53 24) (size 0.6) (drill 0.3) (layers "F.Cu" "B.Cu") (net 6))
 (segment (start 53 24) (end 53 29.62) (width 0.25) (layer "B.Cu") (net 6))
 (segment (start 53 29.62) (end 46 29.62) (width 0.25) (layer "B.Cu") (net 6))
 (gr_rect (start 0 0) (end 60 40) (stroke (width 0.1) (type default)) (fill none) (layer "Edge.Cuts"))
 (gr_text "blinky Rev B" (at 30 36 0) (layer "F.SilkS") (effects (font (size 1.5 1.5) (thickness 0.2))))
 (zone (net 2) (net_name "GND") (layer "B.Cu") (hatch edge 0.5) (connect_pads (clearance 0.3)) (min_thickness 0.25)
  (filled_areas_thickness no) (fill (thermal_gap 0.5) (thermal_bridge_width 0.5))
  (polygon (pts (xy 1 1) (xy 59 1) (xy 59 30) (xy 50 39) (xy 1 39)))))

